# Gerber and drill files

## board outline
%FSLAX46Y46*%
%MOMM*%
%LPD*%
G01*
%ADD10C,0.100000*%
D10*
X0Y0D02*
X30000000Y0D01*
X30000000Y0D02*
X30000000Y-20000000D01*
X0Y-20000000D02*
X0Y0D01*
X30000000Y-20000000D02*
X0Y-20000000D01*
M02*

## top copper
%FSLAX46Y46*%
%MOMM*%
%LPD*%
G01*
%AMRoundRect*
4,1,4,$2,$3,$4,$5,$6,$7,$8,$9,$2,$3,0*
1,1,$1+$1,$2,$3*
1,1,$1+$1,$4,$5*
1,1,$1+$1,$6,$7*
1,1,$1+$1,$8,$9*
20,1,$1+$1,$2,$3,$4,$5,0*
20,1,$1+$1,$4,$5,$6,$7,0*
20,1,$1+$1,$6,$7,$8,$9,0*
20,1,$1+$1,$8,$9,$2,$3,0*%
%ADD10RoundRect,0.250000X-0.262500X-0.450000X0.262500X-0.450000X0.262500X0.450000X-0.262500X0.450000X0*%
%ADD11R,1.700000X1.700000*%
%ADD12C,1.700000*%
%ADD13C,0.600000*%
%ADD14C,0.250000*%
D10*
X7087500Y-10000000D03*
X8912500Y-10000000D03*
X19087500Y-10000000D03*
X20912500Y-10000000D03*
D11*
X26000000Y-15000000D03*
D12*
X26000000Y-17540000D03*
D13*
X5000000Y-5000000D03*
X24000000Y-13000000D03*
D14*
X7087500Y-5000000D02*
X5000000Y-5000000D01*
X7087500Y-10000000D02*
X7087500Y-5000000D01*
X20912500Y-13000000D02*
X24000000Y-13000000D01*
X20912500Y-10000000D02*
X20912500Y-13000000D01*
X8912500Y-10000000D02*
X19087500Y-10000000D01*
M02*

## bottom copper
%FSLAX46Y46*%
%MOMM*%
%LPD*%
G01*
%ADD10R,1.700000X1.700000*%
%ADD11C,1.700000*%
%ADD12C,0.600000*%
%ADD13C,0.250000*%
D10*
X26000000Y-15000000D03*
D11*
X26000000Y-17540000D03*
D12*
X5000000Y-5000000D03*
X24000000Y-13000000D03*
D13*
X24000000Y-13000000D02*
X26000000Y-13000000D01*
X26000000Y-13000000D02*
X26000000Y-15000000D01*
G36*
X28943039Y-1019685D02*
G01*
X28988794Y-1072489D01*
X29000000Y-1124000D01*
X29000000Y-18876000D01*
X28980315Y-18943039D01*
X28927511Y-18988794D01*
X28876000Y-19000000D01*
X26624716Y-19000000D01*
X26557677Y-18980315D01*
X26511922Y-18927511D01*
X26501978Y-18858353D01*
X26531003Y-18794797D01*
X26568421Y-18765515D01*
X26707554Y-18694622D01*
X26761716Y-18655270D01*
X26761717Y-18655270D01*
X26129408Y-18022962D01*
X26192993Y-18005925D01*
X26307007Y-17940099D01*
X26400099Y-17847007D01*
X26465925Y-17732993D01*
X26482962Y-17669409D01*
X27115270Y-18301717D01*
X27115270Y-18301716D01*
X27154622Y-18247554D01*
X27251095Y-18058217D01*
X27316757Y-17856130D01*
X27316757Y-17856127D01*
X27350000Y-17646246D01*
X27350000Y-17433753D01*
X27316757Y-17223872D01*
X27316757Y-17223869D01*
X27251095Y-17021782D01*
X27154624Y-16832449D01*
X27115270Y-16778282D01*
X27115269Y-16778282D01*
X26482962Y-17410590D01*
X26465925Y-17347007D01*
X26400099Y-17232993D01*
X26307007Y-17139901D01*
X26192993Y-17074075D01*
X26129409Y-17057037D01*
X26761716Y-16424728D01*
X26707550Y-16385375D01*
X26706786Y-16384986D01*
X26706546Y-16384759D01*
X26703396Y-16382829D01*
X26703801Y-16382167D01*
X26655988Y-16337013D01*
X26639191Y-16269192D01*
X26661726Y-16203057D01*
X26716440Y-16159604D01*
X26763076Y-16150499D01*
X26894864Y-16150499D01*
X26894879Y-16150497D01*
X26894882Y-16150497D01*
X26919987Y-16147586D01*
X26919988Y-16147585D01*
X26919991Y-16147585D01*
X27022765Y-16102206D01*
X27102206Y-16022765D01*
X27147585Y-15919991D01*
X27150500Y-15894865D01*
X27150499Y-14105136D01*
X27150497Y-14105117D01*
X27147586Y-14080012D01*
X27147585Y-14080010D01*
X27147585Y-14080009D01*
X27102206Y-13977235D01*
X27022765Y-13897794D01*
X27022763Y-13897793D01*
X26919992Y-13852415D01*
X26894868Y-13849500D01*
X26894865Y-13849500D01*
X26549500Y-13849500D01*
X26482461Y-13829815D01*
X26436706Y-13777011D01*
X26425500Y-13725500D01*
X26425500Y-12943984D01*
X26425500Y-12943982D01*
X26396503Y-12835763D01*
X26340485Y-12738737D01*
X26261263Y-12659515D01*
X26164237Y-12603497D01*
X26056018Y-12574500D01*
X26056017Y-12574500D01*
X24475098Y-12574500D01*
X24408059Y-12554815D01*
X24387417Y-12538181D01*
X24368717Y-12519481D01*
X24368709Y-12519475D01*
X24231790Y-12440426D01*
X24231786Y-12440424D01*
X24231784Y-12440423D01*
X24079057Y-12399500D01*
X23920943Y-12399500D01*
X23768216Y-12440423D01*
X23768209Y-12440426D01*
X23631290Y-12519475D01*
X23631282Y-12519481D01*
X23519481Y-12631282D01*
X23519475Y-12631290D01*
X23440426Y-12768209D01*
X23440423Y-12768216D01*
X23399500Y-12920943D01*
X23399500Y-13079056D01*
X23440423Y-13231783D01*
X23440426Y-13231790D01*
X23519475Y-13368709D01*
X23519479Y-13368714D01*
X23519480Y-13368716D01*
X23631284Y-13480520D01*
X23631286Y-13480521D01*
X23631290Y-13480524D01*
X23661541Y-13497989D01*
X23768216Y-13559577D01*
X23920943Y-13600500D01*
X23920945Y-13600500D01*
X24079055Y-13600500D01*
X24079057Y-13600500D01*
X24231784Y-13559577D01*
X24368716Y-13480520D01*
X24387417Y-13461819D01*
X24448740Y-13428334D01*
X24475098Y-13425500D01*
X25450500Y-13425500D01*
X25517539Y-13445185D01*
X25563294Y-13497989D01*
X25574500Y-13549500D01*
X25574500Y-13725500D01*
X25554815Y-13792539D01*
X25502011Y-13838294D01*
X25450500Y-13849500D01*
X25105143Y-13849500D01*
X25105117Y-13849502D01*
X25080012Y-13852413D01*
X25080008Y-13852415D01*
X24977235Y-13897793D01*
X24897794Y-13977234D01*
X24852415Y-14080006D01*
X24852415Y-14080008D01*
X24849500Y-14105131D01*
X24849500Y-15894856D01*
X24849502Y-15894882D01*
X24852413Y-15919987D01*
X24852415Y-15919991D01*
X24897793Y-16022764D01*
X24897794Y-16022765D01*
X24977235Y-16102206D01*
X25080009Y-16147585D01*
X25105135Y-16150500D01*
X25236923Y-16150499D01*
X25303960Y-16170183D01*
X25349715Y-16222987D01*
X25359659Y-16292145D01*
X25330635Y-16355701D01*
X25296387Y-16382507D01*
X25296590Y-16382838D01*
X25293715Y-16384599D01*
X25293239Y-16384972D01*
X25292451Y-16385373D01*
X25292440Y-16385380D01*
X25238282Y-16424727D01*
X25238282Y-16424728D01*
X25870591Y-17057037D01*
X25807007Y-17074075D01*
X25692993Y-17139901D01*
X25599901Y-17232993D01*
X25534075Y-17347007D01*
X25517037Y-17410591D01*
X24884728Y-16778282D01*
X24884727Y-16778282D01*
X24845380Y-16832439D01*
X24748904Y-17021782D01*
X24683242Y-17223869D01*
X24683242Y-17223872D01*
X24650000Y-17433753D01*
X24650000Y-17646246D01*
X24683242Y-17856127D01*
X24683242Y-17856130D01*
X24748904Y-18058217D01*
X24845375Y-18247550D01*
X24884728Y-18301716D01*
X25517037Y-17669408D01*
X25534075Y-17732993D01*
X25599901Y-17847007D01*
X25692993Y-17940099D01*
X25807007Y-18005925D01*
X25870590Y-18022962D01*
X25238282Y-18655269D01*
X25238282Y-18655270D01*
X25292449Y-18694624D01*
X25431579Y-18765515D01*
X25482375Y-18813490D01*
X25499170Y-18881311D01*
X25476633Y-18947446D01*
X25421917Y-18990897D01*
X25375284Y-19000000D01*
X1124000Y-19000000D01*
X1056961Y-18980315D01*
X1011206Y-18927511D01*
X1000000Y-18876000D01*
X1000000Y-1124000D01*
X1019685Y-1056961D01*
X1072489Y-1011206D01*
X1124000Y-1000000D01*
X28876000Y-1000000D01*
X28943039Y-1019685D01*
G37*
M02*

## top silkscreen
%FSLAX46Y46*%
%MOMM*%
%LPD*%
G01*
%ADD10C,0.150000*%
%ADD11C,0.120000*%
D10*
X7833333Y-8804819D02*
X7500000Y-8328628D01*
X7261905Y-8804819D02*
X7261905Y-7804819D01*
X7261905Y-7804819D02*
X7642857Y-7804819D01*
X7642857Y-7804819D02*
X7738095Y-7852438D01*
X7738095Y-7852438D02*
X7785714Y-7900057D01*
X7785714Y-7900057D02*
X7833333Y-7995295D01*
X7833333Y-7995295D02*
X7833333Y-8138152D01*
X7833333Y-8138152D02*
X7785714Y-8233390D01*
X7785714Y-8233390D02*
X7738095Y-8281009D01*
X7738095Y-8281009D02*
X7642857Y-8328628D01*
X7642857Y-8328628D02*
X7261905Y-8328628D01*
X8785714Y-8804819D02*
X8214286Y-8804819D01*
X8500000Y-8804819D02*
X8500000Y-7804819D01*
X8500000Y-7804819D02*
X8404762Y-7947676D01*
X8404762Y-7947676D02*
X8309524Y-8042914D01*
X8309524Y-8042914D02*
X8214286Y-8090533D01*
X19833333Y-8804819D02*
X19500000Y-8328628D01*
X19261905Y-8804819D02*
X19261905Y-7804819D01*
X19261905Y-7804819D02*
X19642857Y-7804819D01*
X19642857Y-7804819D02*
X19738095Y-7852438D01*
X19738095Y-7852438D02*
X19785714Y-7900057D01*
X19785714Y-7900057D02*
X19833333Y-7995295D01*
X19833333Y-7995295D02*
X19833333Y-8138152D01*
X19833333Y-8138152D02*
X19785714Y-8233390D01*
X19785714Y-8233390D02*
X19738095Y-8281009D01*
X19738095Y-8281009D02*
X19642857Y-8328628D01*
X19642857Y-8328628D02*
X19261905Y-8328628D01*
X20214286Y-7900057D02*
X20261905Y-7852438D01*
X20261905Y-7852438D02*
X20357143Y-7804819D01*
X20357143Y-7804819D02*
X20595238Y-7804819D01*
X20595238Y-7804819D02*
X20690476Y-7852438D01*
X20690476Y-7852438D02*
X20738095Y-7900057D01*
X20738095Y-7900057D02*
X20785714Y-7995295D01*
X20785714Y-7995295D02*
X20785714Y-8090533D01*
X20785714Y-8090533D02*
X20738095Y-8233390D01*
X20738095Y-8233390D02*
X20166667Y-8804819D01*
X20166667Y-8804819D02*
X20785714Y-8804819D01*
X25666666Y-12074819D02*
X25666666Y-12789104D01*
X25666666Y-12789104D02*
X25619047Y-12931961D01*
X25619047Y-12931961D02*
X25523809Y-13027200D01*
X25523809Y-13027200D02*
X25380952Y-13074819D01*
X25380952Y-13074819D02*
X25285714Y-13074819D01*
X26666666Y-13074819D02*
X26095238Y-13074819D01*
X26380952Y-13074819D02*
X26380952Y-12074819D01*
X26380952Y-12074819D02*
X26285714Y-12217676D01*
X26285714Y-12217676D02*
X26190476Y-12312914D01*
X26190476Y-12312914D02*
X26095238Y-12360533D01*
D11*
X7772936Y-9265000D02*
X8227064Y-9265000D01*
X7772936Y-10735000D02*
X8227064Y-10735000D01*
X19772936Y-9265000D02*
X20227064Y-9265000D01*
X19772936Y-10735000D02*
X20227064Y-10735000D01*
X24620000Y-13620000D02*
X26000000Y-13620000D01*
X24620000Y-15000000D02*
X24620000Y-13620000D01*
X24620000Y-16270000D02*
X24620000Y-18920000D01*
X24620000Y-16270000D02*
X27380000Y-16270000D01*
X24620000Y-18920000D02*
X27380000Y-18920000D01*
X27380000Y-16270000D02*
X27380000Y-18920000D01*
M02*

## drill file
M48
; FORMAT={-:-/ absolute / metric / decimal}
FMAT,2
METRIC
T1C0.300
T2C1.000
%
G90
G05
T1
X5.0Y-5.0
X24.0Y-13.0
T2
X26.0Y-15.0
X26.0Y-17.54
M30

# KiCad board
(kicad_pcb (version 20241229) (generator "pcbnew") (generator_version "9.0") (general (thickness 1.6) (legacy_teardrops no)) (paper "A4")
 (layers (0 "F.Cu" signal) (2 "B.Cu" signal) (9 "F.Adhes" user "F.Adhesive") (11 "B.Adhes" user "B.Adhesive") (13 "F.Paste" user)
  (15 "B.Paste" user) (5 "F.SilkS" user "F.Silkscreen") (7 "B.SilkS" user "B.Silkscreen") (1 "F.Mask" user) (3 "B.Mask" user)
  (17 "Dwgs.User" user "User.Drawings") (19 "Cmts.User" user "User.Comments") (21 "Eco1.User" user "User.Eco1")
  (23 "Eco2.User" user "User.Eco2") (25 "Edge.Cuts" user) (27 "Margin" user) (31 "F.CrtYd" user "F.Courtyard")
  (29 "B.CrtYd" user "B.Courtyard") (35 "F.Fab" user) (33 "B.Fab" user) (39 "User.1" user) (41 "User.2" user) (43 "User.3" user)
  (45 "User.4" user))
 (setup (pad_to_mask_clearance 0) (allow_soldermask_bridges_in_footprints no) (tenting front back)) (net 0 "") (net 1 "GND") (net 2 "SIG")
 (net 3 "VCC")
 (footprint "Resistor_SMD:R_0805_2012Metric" (layer "F.Cu") (at 8 10)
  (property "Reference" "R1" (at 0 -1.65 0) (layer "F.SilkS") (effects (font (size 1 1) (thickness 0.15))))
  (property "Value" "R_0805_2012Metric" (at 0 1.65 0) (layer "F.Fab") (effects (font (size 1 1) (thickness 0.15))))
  (fp_line (start -0.227064 -0.735) (end 0.227064 -0.735) (stroke (width 0.12) (type solid)) (layer "F.SilkS"))
  (fp_line (start -0.227064 0.735) (end 0.227064 0.735) (stroke (width 0.12) (type solid)) (layer "F.SilkS"))
  (pad "1" smd roundrect (at -0.9125 0) (size 1.025 1.4) (layers "F.Cu" "F.Mask" "F.Paste") (roundrect_rratio 0.243902) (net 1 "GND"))
  (pad "2" smd roundrect (at 0.9125 0) (size 1.025 1.4) (layers "F.Cu" "F.Mask" "F.Paste") (roundrect_rratio 0.243902) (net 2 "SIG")))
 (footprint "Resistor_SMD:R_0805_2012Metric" (layer "F.Cu") (at 20 10)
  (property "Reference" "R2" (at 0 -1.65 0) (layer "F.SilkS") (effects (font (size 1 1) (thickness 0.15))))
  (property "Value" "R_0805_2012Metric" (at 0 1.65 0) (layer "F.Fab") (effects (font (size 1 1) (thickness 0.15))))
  (fp_line (start -0.227064 -0.735) (end 0.227064 -0.735) (stroke (width 0.12) (type solid)) (layer "F.SilkS"))
  (fp_line (start -0.227064 0.735) (end 0.227064 0.735) (stroke (width 0.12) (type solid)) (layer "F.SilkS"))
  (pad "1" smd roundrect (at -0.9125 0) (size 1.025 1.4) (layers "F.Cu" "F.Mask" "F.Paste") (roundrect_rratio 0.243902) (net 2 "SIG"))
  (pad "2" smd roundrect (at 0.9125 0) (size 1.025 1.4) (layers "F.Cu" "F.Mask" "F.Paste") (roundrect_rratio 0.243902) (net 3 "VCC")))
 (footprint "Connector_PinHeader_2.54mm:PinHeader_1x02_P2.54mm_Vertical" (layer "F.Cu") (at 26 15)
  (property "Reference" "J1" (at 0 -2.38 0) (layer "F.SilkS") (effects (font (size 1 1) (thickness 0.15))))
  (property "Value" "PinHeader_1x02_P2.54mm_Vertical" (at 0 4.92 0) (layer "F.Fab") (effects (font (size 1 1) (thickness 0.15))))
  (fp_line (start -1.38 -1.38) (end 0 -1.38) (stroke (width 0.12) (type solid)) (layer "F.SilkS"))
  (fp_line (start -1.38 0) (end -1.38 -1.38) (stroke (width 0.12) (type solid)) (layer "F.SilkS"))
  (fp_line (start -1.38 1.27) (end -1.38 3.92) (stroke (width 0.12) (type solid)) (layer "F.SilkS"))
  (fp_line (start -1.38 1.27) (end 1.38 1.27) (stroke (width 0.12) (type solid)) (layer "F.SilkS"))
  (fp_line (start -1.38 3.92) (end 1.38 3.92) (stroke (width 0.12) (type solid)) (layer "F.SilkS"))
  (fp_line (start 1.38 1.27) (end 1.38 3.92) (stroke (width 0.12) (type solid)) (layer "F.SilkS"))
  (pad "1" thru_hole rect (at 0 0) (size 1.7 1.7) (drill 1) (layers "*.Cu" "*.Mask") (remove_unused_layers no) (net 3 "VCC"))
  (pad "2" thru_hole circle (at 0 2.54) (size 1.7 1.7) (drill 1) (layers "*.Cu" "*.Mask") (remove_unused_layers no) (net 1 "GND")))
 (gr_line (start 0 0) (end 30 0) (stroke (width 0.1) (type default)) (layer "Edge.Cuts"))
 (gr_line (start 30 0) (end 30 20) (stroke (width 0.1) (type default)) (layer "Edge.Cuts"))
 (gr_line (start 0 20) (end 0 0) (stroke (width 0.1) (type default)) (layer "Edge.Cuts"))
 (gr_line (start 30 20) (end 0 20) (stroke (width 0.1) (type default)) (layer "Edge.Cuts"))
 (segment (start 7.0875 5) (end 5 5) (width 0.25) (layer "F.Cu") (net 1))
 (segment (start 7.0875 10) (end 7.0875 5) (width 0.25) (layer "F.Cu") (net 1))
 (via (at 5 5) (size 0.6) (drill 0.3) (layers "F.Cu" "B.Cu") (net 1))
 (segment (start 20.9125 13) (end 24 13) (width 0.25) (layer "F.Cu") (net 3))
 (segment (start 20.9125 10) (end 20.9125 13) (width 0.25) (layer "F.Cu") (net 3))
 (via (at 24 13) (size 0.6) (drill 0.3) (layers "F.Cu" "B.Cu") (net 3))
 (segment (start 24 13) (end 26 13) (width 0.25) (layer "B.Cu") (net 3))
 (segment (start 26 13) (end 26 15) (width 0.25) (layer "B.Cu") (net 3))
 (segment (start 8.9125 10) (end 19.0875 10) (width 0.25) (layer "F.Cu") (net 2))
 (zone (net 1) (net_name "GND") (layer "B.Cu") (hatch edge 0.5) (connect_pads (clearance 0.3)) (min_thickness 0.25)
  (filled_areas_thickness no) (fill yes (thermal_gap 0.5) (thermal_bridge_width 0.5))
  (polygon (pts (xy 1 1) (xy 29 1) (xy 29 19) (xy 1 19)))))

